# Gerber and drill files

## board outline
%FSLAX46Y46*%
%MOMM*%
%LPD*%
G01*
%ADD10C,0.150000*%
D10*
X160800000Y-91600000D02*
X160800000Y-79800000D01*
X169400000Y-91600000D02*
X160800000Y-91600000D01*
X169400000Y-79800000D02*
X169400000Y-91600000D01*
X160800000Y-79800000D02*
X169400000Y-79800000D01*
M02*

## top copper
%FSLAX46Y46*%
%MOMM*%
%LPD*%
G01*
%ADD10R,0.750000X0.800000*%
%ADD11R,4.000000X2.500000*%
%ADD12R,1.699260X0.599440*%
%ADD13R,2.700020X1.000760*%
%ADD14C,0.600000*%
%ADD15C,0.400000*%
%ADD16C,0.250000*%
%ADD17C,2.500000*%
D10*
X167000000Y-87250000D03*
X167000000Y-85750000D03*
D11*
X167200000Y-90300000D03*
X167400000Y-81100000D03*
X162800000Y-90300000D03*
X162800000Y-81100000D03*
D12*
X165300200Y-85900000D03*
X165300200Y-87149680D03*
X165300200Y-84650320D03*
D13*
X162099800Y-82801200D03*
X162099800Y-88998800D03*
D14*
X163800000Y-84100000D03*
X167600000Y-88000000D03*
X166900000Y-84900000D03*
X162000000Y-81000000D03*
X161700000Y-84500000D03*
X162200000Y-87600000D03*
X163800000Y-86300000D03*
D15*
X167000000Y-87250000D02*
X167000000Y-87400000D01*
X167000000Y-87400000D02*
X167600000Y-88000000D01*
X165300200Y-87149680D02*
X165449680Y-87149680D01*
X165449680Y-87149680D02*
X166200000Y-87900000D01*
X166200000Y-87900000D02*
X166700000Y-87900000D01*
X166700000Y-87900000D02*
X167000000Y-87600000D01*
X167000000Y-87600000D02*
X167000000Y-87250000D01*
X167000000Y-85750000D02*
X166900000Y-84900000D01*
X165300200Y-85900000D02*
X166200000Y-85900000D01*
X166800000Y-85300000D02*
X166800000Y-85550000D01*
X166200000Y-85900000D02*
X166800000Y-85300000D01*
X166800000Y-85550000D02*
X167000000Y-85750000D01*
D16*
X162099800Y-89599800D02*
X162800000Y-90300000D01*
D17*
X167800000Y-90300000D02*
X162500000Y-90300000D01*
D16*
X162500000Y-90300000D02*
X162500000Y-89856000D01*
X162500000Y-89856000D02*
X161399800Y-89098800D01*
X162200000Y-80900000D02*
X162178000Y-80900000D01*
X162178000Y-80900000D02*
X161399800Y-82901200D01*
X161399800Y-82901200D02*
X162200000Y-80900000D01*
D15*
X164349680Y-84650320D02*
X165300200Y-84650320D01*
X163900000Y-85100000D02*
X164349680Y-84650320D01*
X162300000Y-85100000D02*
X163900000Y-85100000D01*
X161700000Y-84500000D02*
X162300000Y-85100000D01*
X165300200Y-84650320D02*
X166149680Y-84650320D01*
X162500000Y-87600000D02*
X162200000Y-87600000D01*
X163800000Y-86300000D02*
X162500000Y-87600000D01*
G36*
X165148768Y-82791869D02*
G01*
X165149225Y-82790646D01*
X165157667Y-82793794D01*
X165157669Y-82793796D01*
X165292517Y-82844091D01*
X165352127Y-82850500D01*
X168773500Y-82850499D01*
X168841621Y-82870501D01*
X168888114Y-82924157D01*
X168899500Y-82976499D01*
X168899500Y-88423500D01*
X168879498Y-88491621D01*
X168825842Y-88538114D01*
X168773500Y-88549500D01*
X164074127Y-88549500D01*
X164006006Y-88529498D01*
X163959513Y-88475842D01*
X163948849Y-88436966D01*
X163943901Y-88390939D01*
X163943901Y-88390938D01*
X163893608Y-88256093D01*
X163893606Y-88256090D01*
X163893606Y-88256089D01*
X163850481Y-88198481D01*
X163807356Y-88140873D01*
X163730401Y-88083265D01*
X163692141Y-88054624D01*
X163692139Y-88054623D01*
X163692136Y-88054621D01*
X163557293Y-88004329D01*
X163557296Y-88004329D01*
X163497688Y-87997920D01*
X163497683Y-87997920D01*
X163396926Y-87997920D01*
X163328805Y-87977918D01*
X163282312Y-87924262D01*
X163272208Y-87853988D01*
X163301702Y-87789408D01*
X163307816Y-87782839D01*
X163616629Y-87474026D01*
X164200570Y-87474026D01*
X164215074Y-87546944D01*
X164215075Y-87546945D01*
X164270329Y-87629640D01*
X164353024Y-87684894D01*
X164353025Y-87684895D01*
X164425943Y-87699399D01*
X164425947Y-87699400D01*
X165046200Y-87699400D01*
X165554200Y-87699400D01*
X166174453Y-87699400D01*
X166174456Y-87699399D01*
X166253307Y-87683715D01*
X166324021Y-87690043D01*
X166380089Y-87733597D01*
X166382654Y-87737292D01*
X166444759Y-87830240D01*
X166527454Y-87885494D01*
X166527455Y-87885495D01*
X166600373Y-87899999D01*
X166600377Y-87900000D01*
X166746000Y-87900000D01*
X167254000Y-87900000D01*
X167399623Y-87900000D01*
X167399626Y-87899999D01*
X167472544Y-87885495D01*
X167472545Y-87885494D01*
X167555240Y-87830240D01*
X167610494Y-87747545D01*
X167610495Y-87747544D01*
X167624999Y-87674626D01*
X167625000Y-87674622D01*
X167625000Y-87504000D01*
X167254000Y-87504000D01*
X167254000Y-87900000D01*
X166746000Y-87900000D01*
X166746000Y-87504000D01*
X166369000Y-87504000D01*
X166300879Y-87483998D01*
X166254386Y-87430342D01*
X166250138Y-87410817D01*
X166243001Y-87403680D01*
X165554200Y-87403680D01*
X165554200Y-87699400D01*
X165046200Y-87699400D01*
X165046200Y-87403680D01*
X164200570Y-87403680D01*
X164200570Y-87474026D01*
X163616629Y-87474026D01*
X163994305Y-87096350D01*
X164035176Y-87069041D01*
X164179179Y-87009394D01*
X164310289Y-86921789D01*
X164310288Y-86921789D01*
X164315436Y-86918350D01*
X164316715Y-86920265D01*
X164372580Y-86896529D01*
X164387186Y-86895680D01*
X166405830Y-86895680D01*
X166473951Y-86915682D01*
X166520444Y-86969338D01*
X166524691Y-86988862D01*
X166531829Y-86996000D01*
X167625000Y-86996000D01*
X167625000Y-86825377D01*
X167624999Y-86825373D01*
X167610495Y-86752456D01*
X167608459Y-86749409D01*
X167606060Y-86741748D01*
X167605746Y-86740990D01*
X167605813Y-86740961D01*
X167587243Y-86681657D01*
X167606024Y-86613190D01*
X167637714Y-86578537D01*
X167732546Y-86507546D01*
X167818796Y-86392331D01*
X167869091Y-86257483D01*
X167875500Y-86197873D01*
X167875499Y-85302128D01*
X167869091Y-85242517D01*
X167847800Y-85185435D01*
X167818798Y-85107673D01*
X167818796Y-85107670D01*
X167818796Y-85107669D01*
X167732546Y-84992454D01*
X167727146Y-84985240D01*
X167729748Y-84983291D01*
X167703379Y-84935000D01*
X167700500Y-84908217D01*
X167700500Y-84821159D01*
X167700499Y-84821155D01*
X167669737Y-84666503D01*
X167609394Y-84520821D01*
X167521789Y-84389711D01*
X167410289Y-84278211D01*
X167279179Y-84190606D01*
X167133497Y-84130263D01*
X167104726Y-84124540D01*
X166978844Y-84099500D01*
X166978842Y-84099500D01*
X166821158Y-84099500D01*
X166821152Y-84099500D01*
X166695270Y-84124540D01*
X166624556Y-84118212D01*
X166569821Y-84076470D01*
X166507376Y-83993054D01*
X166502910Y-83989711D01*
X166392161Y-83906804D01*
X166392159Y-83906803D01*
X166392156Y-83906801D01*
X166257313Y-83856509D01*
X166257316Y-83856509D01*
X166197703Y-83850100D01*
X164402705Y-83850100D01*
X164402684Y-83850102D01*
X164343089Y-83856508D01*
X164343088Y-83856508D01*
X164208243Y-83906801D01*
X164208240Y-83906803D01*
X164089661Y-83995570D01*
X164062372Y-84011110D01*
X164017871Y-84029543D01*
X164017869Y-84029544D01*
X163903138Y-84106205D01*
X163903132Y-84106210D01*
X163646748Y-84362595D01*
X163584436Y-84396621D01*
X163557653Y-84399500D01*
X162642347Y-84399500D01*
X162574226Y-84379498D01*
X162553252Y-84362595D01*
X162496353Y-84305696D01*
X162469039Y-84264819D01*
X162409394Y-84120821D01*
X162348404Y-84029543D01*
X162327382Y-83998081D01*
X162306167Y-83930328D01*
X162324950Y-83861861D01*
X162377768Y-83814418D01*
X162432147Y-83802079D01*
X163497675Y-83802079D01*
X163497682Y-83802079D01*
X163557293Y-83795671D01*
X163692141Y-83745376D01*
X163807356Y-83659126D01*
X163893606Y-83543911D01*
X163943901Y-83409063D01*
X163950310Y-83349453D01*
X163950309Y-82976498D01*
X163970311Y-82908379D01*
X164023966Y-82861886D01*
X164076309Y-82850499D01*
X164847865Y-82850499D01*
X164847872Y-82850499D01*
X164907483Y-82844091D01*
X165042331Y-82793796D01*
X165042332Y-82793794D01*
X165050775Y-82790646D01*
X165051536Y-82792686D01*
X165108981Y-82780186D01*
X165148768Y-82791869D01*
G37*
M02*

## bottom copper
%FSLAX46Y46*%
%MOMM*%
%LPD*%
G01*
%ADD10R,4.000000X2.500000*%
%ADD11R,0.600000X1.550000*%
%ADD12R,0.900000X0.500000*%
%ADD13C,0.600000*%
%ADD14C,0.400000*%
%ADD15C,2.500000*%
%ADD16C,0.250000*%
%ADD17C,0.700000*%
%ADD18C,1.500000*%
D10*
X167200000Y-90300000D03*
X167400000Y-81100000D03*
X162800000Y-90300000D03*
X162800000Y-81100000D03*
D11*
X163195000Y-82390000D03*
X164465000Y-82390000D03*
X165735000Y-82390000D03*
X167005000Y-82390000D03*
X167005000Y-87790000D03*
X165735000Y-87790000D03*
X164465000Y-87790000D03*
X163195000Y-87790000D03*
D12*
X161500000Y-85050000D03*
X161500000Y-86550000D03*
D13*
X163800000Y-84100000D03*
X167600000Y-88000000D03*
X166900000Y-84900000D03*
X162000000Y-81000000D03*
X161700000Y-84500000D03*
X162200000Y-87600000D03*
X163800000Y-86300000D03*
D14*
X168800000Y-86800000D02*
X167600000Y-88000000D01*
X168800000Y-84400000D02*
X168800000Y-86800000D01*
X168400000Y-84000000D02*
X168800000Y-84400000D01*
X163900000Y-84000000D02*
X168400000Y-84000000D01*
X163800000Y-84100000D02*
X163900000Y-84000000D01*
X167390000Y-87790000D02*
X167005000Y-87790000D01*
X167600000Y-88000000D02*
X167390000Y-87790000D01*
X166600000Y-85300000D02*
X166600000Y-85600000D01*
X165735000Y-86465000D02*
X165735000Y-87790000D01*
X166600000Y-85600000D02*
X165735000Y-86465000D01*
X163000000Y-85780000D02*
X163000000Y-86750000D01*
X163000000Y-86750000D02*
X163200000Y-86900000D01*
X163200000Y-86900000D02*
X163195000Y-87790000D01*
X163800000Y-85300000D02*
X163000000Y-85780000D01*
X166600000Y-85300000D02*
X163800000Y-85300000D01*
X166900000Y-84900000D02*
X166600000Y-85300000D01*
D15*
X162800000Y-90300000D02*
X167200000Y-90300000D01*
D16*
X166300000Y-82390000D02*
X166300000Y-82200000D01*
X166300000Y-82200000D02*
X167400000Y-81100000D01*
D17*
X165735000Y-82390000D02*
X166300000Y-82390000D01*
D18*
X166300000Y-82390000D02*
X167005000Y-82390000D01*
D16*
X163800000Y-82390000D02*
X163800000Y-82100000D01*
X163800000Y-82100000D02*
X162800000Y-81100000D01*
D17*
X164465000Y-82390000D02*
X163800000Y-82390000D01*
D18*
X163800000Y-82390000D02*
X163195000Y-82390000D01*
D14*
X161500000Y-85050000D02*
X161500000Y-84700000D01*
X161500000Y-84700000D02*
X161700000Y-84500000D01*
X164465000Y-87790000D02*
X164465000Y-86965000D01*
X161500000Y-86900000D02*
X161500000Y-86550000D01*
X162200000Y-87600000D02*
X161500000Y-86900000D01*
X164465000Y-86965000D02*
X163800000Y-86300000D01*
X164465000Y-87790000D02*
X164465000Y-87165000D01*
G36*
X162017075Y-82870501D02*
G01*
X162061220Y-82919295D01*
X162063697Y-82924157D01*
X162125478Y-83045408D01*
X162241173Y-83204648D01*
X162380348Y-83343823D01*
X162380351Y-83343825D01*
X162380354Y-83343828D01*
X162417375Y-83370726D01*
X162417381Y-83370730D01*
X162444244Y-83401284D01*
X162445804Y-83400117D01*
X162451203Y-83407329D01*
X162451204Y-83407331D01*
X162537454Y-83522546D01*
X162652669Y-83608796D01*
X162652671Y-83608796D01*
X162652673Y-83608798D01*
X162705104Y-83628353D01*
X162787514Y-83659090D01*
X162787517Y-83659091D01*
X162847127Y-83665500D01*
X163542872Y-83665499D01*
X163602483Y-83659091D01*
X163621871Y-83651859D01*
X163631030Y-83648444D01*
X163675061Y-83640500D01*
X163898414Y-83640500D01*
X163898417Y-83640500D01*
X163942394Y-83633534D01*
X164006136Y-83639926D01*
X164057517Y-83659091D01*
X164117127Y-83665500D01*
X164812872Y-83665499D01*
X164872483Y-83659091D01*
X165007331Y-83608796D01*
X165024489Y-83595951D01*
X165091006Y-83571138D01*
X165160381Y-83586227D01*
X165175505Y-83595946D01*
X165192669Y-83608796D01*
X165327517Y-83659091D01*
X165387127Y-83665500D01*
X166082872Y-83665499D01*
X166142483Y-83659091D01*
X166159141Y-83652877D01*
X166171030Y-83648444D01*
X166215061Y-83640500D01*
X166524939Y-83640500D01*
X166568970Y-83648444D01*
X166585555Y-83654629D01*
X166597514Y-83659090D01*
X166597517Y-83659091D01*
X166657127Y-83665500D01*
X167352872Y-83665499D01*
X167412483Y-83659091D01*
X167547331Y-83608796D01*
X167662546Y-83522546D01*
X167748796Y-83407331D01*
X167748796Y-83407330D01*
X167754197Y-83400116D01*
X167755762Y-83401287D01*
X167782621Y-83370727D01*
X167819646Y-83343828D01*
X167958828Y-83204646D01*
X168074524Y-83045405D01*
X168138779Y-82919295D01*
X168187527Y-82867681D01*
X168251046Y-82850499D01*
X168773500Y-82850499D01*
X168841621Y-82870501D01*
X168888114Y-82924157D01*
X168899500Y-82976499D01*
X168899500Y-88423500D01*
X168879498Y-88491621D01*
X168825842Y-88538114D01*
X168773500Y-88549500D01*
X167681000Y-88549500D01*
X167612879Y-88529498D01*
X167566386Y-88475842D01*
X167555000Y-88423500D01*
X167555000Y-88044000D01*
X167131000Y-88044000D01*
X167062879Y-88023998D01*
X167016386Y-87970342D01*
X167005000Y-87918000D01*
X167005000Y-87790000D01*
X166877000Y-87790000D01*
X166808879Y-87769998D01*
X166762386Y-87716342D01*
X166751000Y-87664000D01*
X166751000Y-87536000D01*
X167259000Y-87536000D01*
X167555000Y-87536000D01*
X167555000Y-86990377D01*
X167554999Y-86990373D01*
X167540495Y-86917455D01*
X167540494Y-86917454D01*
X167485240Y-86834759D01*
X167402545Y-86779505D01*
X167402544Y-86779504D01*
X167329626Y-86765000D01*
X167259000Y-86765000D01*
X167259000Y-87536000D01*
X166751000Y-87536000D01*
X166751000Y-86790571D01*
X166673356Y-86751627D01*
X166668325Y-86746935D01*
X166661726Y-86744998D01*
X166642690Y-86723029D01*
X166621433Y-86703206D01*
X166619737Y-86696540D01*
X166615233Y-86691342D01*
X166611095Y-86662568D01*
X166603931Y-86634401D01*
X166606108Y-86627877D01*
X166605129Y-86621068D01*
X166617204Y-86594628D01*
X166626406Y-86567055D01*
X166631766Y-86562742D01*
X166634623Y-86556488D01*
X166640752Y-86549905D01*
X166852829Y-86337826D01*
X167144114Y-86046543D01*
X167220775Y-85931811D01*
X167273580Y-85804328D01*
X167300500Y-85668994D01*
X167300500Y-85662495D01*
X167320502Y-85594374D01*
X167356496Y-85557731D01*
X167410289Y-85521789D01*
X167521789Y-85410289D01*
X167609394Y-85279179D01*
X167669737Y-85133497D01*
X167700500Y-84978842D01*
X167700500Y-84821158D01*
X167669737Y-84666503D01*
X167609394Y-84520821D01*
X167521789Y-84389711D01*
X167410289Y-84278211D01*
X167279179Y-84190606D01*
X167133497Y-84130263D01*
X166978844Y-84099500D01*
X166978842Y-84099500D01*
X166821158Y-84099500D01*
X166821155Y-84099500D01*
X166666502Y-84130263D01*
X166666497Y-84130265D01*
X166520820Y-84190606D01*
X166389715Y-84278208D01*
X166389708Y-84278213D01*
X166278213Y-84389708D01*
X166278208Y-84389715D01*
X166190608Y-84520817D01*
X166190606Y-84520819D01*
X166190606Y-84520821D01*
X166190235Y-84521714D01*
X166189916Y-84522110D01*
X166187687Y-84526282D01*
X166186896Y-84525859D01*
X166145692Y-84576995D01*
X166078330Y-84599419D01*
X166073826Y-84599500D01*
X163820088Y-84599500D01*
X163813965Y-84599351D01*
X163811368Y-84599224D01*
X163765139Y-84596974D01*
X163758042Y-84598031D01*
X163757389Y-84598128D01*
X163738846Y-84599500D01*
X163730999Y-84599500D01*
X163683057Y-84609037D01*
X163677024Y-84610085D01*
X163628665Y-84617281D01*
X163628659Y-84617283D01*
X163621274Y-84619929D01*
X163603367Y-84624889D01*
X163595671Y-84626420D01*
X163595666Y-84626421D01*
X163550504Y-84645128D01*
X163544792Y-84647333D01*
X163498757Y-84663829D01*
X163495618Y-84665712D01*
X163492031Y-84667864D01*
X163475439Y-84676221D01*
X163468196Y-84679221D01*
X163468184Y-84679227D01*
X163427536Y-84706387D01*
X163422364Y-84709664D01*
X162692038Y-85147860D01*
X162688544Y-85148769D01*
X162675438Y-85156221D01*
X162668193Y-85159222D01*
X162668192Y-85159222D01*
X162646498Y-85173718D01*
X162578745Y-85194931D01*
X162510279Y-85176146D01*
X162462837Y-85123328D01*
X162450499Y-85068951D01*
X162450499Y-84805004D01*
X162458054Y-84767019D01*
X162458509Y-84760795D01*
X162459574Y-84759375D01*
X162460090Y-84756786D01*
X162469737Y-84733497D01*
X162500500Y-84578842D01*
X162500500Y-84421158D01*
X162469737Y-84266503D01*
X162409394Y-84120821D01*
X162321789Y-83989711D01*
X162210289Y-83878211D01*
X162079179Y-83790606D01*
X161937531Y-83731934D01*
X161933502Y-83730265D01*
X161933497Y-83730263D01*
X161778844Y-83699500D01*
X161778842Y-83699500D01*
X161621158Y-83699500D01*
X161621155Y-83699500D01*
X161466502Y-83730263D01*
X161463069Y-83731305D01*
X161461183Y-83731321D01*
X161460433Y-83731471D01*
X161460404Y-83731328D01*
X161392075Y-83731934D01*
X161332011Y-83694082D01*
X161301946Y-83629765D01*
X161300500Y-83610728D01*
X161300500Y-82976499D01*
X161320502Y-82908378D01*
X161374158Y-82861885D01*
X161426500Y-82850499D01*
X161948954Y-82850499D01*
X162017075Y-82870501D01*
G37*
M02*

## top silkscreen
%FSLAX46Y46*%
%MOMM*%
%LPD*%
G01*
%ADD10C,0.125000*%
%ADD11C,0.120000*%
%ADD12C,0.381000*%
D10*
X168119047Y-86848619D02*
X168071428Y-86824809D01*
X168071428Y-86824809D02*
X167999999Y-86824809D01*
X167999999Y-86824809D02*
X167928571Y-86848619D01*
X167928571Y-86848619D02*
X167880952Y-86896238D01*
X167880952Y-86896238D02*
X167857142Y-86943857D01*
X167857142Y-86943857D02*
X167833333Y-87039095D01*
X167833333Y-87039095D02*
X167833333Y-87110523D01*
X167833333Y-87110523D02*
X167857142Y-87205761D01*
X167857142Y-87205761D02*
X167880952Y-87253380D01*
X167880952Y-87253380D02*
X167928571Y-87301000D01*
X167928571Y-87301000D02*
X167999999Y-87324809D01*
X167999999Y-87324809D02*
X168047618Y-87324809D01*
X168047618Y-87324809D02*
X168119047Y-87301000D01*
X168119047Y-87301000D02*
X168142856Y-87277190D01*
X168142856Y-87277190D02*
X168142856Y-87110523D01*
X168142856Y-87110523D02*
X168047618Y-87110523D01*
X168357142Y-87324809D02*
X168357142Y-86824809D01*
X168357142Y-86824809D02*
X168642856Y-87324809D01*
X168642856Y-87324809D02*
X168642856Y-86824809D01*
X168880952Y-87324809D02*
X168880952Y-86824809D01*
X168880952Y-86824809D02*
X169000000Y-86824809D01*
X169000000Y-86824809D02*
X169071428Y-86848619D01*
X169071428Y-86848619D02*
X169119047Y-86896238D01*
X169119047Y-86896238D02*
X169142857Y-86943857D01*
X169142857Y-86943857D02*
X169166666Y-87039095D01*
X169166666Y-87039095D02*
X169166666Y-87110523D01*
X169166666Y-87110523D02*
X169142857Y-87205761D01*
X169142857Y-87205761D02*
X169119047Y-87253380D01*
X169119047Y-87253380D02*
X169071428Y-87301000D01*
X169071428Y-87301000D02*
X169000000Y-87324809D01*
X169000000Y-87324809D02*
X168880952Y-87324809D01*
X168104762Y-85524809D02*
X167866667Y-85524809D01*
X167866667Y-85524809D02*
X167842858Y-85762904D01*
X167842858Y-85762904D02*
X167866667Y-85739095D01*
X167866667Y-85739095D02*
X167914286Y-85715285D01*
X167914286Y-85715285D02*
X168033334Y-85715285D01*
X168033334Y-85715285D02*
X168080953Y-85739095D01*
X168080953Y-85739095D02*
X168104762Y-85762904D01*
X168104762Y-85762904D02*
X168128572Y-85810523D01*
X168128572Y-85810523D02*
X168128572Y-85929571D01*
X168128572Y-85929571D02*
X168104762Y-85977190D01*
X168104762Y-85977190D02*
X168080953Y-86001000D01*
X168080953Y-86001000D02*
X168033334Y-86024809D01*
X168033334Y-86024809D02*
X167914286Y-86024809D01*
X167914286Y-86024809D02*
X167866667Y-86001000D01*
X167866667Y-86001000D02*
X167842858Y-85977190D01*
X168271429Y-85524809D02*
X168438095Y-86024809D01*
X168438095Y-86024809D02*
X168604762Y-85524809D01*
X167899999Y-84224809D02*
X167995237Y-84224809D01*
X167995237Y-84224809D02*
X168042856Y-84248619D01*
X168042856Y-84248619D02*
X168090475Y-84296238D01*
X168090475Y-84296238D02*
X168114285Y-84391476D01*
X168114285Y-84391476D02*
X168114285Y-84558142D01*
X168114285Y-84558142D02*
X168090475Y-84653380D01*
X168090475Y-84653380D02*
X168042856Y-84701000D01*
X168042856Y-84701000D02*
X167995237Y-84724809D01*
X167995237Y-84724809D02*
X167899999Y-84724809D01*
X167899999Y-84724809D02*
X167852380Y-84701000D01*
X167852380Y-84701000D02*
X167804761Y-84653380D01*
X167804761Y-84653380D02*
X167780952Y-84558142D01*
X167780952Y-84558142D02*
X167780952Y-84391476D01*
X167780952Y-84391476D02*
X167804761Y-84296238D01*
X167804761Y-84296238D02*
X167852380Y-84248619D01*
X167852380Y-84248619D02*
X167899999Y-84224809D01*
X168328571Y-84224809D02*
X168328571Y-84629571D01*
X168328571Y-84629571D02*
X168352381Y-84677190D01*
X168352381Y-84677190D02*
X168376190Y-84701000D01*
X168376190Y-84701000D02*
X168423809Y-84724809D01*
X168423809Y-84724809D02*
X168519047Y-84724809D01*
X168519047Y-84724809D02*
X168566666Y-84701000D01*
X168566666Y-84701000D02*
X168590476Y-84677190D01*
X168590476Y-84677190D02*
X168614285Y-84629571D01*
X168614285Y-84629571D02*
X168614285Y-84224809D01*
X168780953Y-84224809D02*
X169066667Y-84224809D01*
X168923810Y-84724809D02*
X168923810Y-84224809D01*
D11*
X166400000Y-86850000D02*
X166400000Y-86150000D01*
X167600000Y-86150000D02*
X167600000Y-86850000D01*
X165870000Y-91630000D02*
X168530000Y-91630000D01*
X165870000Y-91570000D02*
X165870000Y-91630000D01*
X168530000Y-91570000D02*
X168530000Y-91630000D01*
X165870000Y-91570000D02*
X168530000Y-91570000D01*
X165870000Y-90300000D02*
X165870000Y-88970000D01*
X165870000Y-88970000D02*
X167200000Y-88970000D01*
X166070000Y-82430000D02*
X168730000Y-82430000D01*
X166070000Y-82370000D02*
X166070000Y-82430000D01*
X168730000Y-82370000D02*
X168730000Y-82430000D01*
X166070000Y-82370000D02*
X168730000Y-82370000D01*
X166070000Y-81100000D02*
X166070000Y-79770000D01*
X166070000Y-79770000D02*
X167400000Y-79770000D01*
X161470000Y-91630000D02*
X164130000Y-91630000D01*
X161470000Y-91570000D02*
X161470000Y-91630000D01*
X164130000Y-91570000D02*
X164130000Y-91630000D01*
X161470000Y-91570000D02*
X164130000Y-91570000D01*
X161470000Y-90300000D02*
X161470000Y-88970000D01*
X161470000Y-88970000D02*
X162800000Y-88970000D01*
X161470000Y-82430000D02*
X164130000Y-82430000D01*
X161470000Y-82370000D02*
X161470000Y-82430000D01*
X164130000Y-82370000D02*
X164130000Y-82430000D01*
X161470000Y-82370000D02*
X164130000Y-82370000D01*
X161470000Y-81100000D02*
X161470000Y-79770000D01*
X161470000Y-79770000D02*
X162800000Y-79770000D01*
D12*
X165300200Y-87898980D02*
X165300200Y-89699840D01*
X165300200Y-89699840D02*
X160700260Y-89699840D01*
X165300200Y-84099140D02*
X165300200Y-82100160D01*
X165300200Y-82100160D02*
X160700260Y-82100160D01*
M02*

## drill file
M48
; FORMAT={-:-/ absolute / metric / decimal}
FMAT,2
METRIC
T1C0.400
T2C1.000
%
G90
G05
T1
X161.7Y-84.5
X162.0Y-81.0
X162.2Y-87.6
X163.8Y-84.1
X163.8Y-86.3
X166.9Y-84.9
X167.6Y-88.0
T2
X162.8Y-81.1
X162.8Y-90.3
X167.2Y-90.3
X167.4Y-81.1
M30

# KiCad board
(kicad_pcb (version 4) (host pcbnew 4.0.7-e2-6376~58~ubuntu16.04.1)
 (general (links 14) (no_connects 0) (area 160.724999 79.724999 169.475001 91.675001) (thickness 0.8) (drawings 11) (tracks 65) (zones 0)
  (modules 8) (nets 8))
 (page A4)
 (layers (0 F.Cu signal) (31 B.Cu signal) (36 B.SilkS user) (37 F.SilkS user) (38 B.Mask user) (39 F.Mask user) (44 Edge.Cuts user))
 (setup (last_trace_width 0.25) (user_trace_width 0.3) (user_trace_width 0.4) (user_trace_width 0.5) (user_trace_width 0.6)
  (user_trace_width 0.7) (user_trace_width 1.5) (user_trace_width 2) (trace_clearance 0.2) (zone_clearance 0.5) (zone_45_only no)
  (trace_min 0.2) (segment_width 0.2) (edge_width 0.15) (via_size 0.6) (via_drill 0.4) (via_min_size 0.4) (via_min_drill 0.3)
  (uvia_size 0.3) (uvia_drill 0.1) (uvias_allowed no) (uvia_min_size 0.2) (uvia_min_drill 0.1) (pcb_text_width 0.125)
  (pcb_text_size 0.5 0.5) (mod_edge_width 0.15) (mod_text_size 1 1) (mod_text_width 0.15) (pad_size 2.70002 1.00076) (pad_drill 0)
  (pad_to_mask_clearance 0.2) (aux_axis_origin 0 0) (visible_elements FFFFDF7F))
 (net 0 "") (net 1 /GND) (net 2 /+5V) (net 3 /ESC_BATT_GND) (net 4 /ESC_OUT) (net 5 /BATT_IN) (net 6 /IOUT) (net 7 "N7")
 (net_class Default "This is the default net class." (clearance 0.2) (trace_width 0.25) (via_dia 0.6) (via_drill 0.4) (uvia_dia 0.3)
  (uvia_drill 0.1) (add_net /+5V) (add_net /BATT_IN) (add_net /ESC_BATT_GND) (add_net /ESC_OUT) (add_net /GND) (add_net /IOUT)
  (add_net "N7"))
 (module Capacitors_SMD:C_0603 (layer F.Cu) (at 167 86.5 270)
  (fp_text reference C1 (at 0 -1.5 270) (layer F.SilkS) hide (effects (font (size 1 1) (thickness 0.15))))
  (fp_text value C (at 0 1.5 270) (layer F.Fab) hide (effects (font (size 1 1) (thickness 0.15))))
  (fp_line (start 0.35 0.6) (end -0.35 0.6) (layer F.SilkS) (width 0.12))
  (fp_line (start -0.35 -0.6) (end 0.35 -0.6) (layer F.SilkS) (width 0.12))
  (pad 2 smd rect (at 0.75 0 270) (size 0.8 0.75) (layers F.Cu F.Mask) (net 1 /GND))
  (pad 1 smd rect (at -0.75 0 270) (size 0.8 0.75) (layers F.Cu F.Mask) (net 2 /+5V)))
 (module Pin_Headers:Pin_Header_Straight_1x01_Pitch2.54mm (layer F.Cu) (at 167.2 90.3)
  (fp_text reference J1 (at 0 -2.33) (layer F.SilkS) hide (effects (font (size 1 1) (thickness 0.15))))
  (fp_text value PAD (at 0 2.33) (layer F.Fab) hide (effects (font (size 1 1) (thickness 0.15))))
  (fp_line (start -1.33 1.33) (end 1.33 1.33) (layer F.SilkS) (width 0.12))
  (fp_line (start -1.33 1.27) (end -1.33 1.33) (layer F.SilkS) (width 0.12))
  (fp_line (start 1.33 1.27) (end 1.33 1.33) (layer F.SilkS) (width 0.12))
  (fp_line (start -1.33 1.27) (end 1.33 1.27) (layer F.SilkS) (width 0.12))
  (fp_line (start -1.33 0) (end -1.33 -1.33) (layer F.SilkS) (width 0.12))
  (fp_line (start -1.33 -1.33) (end 0 -1.33) (layer F.SilkS) (width 0.12))
  (pad 1 thru_hole rect (at 0 0) (size 4 2.5) (drill 1) (layers *.Cu *.Mask) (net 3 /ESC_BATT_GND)))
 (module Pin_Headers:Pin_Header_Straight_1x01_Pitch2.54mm (layer F.Cu) (at 167.4 81.1)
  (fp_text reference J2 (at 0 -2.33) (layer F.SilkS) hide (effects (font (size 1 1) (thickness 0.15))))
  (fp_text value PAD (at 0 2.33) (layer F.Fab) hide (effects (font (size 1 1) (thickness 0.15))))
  (fp_line (start -1.33 1.33) (end 1.33 1.33) (layer F.SilkS) (width 0.12))
  (fp_line (start -1.33 1.27) (end -1.33 1.33) (layer F.SilkS) (width 0.12))
  (fp_line (start 1.33 1.27) (end 1.33 1.33) (layer F.SilkS) (width 0.12))
  (fp_line (start -1.33 1.27) (end 1.33 1.27) (layer F.SilkS) (width 0.12))
  (fp_line (start -1.33 0) (end -1.33 -1.33) (layer F.SilkS) (width 0.12))
  (fp_line (start -1.33 -1.33) (end 0 -1.33) (layer F.SilkS) (width 0.12))
  (pad 1 thru_hole rect (at 0 0) (size 4 2.5) (drill 1) (layers *.Cu *.Mask) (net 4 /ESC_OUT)))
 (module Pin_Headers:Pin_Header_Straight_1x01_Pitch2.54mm (layer F.Cu) (at 162.8 90.3)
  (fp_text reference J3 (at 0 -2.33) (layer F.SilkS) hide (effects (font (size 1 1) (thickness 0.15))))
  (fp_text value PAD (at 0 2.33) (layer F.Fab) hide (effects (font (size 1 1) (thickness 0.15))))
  (fp_line (start -1.33 1.33) (end 1.33 1.33) (layer F.SilkS) (width 0.12))
  (fp_line (start -1.33 1.27) (end -1.33 1.33) (layer F.SilkS) (width 0.12))
  (fp_line (start 1.33 1.27) (end 1.33 1.33) (layer F.SilkS) (width 0.12))
  (fp_line (start -1.33 1.27) (end 1.33 1.27) (layer F.SilkS) (width 0.12))
  (fp_line (start -1.33 0) (end -1.33 -1.33) (layer F.SilkS) (width 0.12))
  (fp_line (start -1.33 -1.33) (end 0 -1.33) (layer F.SilkS) (width 0.12))
  (pad 1 thru_hole rect (at 0 0) (size 4 2.5) (drill 1) (layers *.Cu *.Mask) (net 3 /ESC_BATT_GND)))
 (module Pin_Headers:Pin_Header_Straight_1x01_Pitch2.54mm (layer F.Cu) (at 162.8 81.1)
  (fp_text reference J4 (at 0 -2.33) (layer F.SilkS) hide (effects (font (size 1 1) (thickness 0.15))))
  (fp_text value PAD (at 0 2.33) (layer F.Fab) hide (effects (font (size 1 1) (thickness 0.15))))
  (fp_line (start -1.33 1.33) (end 1.33 1.33) (layer F.SilkS) (width 0.12))
  (fp_line (start -1.33 1.27) (end -1.33 1.33) (layer F.SilkS) (width 0.12))
  (fp_line (start 1.33 1.27) (end 1.33 1.33) (layer F.SilkS) (width 0.12))
  (fp_line (start -1.33 1.27) (end 1.33 1.27) (layer F.SilkS) (width 0.12))
  (fp_line (start -1.33 0) (end -1.33 -1.33) (layer F.SilkS) (width 0.12))
  (fp_line (start -1.33 -1.33) (end 0 -1.33) (layer F.SilkS) (width 0.12))
  (pad 1 thru_hole rect (at 0 0) (size 4 2.5) (drill 1) (layers *.Cu *.Mask) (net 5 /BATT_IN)))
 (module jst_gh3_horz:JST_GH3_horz (layer F.Cu) (at 163.7 85.9)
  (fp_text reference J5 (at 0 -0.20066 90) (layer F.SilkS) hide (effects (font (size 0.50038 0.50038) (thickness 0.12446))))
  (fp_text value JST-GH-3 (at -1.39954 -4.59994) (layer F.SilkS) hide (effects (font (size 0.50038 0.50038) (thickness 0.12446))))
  (fp_line (start 1.6002 1.99898) (end 1.6002 3.79984) (layer F.SilkS) (width 0.381))
  (fp_line (start 1.6002 3.79984) (end -2.99974 3.79984) (layer F.SilkS) (width 0.381))
  (fp_line (start 1.6002 -1.80086) (end 1.6002 -3.79984) (layer F.SilkS) (width 0.381))
  (fp_line (start 1.6002 -3.79984) (end -2.99974 -3.79984) (layer F.SilkS) (width 0.381))
  (pad 2 smd rect (at 1.6002 0 270) (size 0.59944 1.69926) (layers F.Cu F.Mask) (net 2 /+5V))
  (pad 3 smd rect (at 1.6002 1.24968 270) (size 0.59944 1.69926) (layers F.Cu F.Mask) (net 1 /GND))
  (pad 1 smd rect (at 1.6002 -1.24968 270) (size 0.59944 1.69926) (layers F.Cu F.Mask) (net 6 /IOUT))
  (pad "" smd rect (at -1.6002 -3.0988) (size 2.70002 1.00076) (layers F.Cu F.Mask) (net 5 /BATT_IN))
  (pad "" smd rect (at -1.6002 3.0988) (size 2.70002 1.00076) (layers F.Cu F.Mask) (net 3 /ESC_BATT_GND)))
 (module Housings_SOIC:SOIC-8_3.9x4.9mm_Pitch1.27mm (layer B.Cu) (at 165.1 85.09 270)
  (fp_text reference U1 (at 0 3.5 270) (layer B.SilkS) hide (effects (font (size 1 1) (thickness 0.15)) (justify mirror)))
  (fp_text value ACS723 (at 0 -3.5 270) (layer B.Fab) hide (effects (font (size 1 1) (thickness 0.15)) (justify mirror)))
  (pad 1 smd rect (at -2.7 1.905 270) (size 1.55 0.6) (layers B.Cu B.Mask) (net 5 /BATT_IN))
  (pad 2 smd rect (at -2.7 0.635 270) (size 1.55 0.6) (layers B.Cu B.Mask) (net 5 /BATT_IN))
  (pad 3 smd rect (at -2.7 -0.635 270) (size 1.55 0.6) (layers B.Cu B.Mask) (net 4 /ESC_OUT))
  (pad 4 smd rect (at -2.7 -1.905 270) (size 1.55 0.6) (layers B.Cu B.Mask) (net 4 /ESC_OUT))
  (pad 5 smd rect (at 2.7 -1.905 270) (size 1.55 0.6) (layers B.Cu B.Mask) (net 1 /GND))
  (pad 6 smd rect (at 2.7 -0.635 270) (size 1.55 0.6) (layers B.Cu B.Mask) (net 2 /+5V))
  (pad 7 smd rect (at 2.7 0.635 270) (size 1.55 0.6) (layers B.Cu B.Mask) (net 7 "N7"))
  (pad 8 smd rect (at 2.7 1.905 270) (size 1.55 0.6) (layers B.Cu B.Mask) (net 2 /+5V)))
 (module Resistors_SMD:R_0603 (layer B.Cu) (at 161.5 85.8 270)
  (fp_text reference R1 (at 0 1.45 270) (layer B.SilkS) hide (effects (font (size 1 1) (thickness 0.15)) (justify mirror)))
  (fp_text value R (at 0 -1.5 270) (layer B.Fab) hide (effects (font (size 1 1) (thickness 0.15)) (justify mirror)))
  (pad 1 smd rect (at -0.75 0 270) (size 0.5 0.9) (layers B.Cu B.Mask) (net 6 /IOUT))
  (pad 2 smd rect (at 0.75 0 270) (size 0.5 0.9) (layers B.Cu B.Mask) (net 7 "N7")))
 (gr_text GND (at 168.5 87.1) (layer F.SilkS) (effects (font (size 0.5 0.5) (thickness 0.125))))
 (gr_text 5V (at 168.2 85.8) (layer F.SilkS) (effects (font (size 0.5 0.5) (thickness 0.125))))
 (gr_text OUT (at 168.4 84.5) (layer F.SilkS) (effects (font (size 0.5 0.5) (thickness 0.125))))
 (gr_line (start 160.8 91.6) (end 160.8 79.8) (angle 90) (layer Edge.Cuts) (width 0.15))
 (gr_line (start 169.4 91.6) (end 160.8 91.6) (angle 90) (layer Edge.Cuts) (width 0.15))
 (gr_line (start 169.4 79.8) (end 169.4 91.6) (angle 90) (layer Edge.Cuts) (width 0.15))
 (gr_line (start 160.8 79.8) (end 169.4 79.8) (angle 90) (layer Edge.Cuts) (width 0.15))
 (segment (start 168.8 86.8) (end 167.6 88) (width 0.4) (layer B.Cu) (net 1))
 (segment (start 168.8 84.4) (end 168.8 86.8) (width 0.4) (layer B.Cu) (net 1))
 (segment (start 168.4 84) (end 168.8 84.4) (width 0.4) (layer B.Cu) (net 1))
 (segment (start 163.9 84) (end 168.4 84) (width 0.4) (layer B.Cu) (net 1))
 (segment (start 163.8 84.1) (end 163.9 84) (width 0.4) (layer B.Cu) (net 1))
 (via (at 163.8 84.1) (size 0.6) (drill 0.4) (layers F.Cu B.Cu) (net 1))
 (segment (start 167 87.25) (end 167 87.4) (width 0.4) (layer F.Cu) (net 1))
 (segment (start 167 87.4) (end 167.6 88) (width 0.4) (layer F.Cu) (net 1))
 (via (at 167.6 88) (size 0.6) (drill 0.4) (layers F.Cu B.Cu) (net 1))
 (segment (start 167.39 87.79) (end 167.005 87.79) (width 0.4) (layer B.Cu) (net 1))
 (segment (start 167.6 88) (end 167.39 87.79) (width 0.4) (layer B.Cu) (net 1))
 (segment (start 165.3002 87.14968) (end 165.44968 87.14968) (width 0.4) (layer F.Cu) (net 1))
 (segment (start 165.44968 87.14968) (end 166.2 87.9) (width 0.4) (layer F.Cu) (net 1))
 (segment (start 166.2 87.9) (end 166.7 87.9) (width 0.4) (layer F.Cu) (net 1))
 (segment (start 166.7 87.9) (end 167 87.6) (width 0.4) (layer F.Cu) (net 1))
 (segment (start 167 87.6) (end 167 87.25) (width 0.4) (layer F.Cu) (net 1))
 (segment (start 166.6 85.3) (end 166.6 85.6) (width 0.4) (layer B.Cu) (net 2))
 (segment (start 165.735 86.465) (end 165.735 87.79) (width 0.4) (layer B.Cu) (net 2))
 (segment (start 166.6 85.6) (end 165.735 86.465) (width 0.4) (layer B.Cu) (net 2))
 (segment (start 167 85.75) (end 166.9 84.9) (width 0.4) (layer F.Cu) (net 2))
 (segment (start 163 85.78) (end 163 86.75) (width 0.4) (layer B.Cu) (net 2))
 (segment (start 163 86.75) (end 163.2 86.9) (width 0.4) (layer B.Cu) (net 2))
 (segment (start 163.2 86.9) (end 163.195 87.79) (width 0.4) (layer B.Cu) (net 2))
 (segment (start 163.8 85.3) (end 163 85.78) (width 0.4) (layer B.Cu) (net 2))
 (segment (start 166.6 85.3) (end 163.8 85.3) (width 0.4) (layer B.Cu) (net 2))
 (segment (start 166.9 84.9) (end 166.6 85.3) (width 0.4) (layer B.Cu) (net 2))
 (via (at 166.9 84.9) (size 0.6) (drill 0.4) (layers F.Cu B.Cu) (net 2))
 (segment (start 165.3002 85.9) (end 166.2 85.9) (width 0.4) (layer F.Cu) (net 2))
 (segment (start 166.8 85.3) (end 166.8 85.55) (width 0.4) (layer F.Cu) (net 2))
 (segment (start 166.2 85.9) (end 166.8 85.3) (width 0.4) (layer F.Cu) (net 2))
 (segment (start 166.8 85.55) (end 167 85.75) (width 0.4) (layer F.Cu) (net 2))
 (segment (start 162.8 90.3) (end 167.2 90.3) (width 2.5) (layer B.Cu) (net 3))
 (segment (start 162.0998 89.5998) (end 162.8 90.3) (width 0.25) (layer F.Cu) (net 3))
 (segment (start 167.8 90.3) (end 162.5 90.3) (width 2.5) (layer F.Cu) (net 3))
 (segment (start 162.5 90.3) (end 162.5 89.856) (width 0.25) (layer F.Cu) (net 3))
 (segment (start 162.5 89.856) (end 161.3998 89.0988) (width 0.25) (layer F.Cu) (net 3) (status 20))
 (segment (start 166.3 82.39) (end 166.3 82.2) (width 0.25) (layer B.Cu) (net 4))
 (segment (start 166.3 82.2) (end 167.4 81.1) (width 0.25) (layer B.Cu) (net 4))
 (segment (start 165.735 82.39) (end 166.3 82.39) (width 0.7) (layer B.Cu) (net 4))
 (segment (start 166.3 82.39) (end 167.005 82.39) (width 1.5) (layer B.Cu) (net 4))
 (segment (start 163.8 82.39) (end 163.8 82.1) (width 0.25) (layer B.Cu) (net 5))
 (segment (start 163.8 82.1) (end 162.8 81.1) (width 0.25) (layer B.Cu) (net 5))
 (segment (start 164.465 82.39) (end 163.8 82.39) (width 0.7) (layer B.Cu) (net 5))
 (segment (start 163.8 82.39) (end 163.195 82.39) (width 1.5) (layer B.Cu) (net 5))
 (via (at 162 81) (size 0.6) (drill 0.4) (layers F.Cu B.Cu) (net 5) (status 30))
 (segment (start 162.2 80.9) (end 162.178 80.9) (width 0.25) (layer F.Cu) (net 5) (status 30))
 (segment (start 162.178 80.9) (end 161.3998 82.9012) (width 0.25) (layer F.Cu) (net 5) (status 20))
 (segment (start 161.3998 82.9012) (end 162.2 80.9) (width 0.25) (layer F.Cu) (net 5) (status 10))
 (segment (start 161.5 85.05) (end 161.5 84.7) (width 0.4) (layer B.Cu) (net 6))
 (segment (start 164.34968 84.65032) (end 165.3002 84.65032) (width 0.4) (layer F.Cu) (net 6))
 (segment (start 163.9 85.1) (end 164.34968 84.65032) (width 0.4) (layer F.Cu) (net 6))
 (segment (start 162.3 85.1) (end 163.9 85.1) (width 0.4) (layer F.Cu) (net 6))
 (segment (start 161.7 84.5) (end 162.3 85.1) (width 0.4) (layer F.Cu) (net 6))
 (via (at 161.7 84.5) (size 0.6) (drill 0.4) (layers F.Cu B.Cu) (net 6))
 (segment (start 161.5 84.7) (end 161.7 84.5) (width 0.4) (layer B.Cu) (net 6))
 (segment (start 165.3002 84.65032) (end 166.14968 84.65032) (width 0.4) (layer F.Cu) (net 6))
 (segment (start 164.465 87.79) (end 164.465 86.965) (width 0.4) (layer B.Cu) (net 7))
 (segment (start 161.5 86.9) (end 161.5 86.55) (width 0.4) (layer B.Cu) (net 7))
 (segment (start 162.2 87.6) (end 161.5 86.9) (width 0.4) (layer B.Cu) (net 7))
 (via (at 162.2 87.6) (size 0.6) (drill 0.4) (layers F.Cu B.Cu) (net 7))
 (segment (start 162.5 87.6) (end 162.2 87.6) (width 0.4) (layer F.Cu) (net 7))
 (segment (start 163.8 86.3) (end 162.5 87.6) (width 0.4) (layer F.Cu) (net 7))
 (via (at 163.8 86.3) (size 0.6) (drill 0.4) (layers F.Cu B.Cu) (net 7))
 (segment (start 164.465 86.965) (end 163.8 86.3) (width 0.4) (layer B.Cu) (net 7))
 (segment (start 164.465 87.79) (end 164.465 87.165) (width 0.4) (layer B.Cu) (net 7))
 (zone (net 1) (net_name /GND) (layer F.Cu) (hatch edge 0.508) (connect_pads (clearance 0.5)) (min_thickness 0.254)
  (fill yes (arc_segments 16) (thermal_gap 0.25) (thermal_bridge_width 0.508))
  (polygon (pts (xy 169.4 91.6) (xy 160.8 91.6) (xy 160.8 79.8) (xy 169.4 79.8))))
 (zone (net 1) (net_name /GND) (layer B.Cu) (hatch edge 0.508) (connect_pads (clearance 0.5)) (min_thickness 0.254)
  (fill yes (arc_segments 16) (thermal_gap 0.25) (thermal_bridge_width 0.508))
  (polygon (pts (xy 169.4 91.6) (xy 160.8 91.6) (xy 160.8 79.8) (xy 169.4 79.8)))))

